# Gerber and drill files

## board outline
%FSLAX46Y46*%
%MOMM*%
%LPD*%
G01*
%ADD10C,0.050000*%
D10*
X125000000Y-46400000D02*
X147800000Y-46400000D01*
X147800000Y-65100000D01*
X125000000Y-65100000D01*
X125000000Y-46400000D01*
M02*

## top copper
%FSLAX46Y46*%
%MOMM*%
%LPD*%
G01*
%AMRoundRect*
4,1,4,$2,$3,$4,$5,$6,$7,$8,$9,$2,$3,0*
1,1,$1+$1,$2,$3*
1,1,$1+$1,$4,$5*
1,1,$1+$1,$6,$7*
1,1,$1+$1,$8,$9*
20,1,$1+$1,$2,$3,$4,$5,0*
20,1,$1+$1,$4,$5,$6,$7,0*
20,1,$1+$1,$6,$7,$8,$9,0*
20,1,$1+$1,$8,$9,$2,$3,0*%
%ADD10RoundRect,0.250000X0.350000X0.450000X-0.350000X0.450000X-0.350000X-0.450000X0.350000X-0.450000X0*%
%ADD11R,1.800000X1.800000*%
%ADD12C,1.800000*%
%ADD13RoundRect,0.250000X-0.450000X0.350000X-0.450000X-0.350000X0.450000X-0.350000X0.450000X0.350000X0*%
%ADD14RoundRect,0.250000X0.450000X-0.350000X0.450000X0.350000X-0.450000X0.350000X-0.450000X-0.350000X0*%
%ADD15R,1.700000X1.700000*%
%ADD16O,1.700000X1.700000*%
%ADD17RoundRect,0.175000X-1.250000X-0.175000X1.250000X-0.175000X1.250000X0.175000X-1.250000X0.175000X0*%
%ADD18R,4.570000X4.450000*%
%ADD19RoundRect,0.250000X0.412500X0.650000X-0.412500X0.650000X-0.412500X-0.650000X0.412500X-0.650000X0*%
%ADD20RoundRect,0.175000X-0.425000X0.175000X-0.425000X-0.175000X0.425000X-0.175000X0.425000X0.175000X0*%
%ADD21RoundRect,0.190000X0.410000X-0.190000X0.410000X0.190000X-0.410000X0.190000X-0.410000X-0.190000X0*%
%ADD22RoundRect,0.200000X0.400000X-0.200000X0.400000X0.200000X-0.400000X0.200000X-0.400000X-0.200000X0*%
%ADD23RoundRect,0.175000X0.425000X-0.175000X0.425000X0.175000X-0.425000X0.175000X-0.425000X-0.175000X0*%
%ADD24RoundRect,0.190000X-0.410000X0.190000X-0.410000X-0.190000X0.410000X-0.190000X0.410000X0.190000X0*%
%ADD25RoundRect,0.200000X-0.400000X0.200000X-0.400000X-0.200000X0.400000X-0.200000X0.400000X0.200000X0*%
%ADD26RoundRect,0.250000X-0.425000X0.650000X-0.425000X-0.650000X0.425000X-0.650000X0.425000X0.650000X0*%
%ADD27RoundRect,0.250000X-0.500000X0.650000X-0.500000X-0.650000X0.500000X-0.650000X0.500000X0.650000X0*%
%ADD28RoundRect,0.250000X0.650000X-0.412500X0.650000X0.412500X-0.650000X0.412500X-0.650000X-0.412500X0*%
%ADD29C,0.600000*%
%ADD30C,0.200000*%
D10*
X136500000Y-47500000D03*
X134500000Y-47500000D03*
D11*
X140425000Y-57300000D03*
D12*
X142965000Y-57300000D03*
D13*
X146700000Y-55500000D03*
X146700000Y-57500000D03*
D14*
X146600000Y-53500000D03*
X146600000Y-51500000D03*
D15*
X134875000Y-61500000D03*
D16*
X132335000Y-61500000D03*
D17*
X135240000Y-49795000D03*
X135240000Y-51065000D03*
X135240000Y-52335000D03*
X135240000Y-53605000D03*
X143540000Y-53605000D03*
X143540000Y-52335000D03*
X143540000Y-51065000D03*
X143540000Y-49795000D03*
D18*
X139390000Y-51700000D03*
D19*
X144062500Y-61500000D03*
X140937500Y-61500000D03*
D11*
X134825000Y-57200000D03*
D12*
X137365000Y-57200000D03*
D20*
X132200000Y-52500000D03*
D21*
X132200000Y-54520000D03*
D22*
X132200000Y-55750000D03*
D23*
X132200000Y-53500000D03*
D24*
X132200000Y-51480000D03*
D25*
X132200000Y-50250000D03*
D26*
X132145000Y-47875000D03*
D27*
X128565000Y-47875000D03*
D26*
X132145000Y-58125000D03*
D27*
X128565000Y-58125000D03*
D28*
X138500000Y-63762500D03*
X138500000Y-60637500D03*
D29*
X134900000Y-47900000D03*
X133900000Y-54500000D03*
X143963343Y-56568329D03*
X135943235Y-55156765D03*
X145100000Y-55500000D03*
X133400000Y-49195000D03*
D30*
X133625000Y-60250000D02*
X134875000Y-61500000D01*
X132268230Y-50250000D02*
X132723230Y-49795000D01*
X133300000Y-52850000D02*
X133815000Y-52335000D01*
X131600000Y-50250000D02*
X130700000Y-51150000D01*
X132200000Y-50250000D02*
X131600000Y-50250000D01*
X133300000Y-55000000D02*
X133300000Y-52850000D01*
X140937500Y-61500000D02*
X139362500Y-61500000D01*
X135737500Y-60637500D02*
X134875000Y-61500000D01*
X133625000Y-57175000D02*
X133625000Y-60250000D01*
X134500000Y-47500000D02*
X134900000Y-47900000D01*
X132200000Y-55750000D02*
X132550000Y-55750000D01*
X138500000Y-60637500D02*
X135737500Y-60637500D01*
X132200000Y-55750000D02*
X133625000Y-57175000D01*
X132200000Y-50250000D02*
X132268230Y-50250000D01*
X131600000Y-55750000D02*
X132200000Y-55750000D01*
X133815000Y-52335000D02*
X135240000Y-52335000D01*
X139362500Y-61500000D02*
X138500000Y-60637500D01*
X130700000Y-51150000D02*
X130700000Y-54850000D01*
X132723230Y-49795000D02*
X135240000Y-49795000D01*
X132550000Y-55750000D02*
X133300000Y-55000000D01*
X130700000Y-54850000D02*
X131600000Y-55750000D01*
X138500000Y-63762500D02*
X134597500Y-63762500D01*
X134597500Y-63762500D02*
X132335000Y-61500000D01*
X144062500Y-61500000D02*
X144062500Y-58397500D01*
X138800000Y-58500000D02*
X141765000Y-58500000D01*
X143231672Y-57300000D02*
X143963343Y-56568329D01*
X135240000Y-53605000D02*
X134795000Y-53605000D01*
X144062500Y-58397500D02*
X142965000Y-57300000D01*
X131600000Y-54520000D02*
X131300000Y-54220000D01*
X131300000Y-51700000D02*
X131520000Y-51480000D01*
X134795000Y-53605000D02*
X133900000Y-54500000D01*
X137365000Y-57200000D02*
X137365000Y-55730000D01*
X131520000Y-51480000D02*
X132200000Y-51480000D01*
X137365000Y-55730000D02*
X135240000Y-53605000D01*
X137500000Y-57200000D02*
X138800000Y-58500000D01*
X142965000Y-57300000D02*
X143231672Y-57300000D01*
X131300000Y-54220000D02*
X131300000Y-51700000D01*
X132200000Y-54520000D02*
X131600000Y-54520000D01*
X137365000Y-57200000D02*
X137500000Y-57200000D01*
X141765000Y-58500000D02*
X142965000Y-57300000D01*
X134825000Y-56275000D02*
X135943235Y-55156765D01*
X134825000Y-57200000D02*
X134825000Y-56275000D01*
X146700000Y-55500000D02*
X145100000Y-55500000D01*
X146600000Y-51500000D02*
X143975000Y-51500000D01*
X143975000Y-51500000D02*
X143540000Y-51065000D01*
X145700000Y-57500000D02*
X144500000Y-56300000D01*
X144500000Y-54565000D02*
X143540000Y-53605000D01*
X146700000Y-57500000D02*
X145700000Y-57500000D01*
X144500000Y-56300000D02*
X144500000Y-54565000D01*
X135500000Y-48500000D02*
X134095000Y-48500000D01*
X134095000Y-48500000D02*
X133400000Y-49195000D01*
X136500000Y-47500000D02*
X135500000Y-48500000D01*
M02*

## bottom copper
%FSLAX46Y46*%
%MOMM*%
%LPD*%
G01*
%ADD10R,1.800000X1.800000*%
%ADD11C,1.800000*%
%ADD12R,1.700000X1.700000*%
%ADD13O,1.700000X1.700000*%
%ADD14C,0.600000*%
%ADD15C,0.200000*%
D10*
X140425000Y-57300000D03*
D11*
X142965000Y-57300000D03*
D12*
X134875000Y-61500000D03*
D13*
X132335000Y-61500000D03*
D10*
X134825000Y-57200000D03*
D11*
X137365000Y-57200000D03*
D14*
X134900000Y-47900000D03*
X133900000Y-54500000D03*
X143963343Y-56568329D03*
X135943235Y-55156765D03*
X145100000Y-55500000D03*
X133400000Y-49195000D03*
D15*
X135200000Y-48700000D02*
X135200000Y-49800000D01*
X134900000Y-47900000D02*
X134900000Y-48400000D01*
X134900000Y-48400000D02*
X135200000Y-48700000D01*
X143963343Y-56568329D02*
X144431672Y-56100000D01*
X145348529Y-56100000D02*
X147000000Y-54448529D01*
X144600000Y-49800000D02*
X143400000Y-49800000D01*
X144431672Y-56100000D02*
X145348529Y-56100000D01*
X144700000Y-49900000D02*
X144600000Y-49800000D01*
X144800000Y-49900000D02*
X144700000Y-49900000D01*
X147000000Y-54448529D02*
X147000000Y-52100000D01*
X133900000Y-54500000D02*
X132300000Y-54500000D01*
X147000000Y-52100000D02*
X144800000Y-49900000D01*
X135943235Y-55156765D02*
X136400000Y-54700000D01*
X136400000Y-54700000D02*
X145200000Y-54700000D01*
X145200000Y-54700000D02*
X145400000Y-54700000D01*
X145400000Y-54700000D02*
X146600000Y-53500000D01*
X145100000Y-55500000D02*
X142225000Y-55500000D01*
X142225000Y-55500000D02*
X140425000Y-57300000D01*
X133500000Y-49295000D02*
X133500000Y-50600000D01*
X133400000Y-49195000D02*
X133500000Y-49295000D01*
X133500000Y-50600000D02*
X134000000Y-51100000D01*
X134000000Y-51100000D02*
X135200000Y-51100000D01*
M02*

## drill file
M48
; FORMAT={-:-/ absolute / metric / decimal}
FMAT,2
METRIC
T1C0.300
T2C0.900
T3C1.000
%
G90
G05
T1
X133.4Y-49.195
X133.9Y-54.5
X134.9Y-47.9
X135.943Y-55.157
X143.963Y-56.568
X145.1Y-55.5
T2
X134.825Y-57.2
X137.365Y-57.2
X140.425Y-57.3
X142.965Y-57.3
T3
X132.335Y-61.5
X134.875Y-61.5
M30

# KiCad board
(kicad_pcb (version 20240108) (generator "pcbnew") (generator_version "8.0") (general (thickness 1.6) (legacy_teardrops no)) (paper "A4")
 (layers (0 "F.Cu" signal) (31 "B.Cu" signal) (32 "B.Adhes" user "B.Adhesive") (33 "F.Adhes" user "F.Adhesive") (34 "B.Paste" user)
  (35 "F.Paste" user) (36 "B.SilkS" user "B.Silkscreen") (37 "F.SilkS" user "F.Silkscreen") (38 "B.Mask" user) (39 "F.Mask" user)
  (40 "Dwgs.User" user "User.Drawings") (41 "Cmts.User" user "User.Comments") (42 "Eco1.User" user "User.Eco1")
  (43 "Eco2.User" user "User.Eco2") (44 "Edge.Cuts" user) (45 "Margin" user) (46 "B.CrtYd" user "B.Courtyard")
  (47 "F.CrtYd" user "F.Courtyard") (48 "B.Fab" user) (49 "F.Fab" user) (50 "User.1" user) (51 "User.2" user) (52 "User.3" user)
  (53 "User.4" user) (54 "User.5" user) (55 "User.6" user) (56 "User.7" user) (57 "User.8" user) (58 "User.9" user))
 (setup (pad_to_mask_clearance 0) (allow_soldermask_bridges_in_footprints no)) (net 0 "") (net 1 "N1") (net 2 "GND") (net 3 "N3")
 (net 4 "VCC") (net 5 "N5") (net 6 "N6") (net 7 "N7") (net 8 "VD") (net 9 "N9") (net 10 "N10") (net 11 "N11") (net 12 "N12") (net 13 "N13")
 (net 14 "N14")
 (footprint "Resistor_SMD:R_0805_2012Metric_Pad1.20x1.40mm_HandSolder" (layer "F.Cu") (at 135.5 47.5 180)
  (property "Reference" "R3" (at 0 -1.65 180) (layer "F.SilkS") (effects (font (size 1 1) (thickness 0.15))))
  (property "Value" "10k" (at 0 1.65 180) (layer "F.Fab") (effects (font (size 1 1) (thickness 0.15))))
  (pad "1" smd roundrect (at -1 0 180) (size 1.2 1.4) (layers "F.Cu" "F.Paste" "F.Mask") (roundrect_rratio 0.208333) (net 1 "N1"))
  (pad "2" smd roundrect (at 1 0 180) (size 1.2 1.4) (layers "F.Cu" "F.Paste" "F.Mask") (roundrect_rratio 0.208333) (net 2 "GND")))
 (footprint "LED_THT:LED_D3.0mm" (layer "F.Cu") (at 140.425 57.3)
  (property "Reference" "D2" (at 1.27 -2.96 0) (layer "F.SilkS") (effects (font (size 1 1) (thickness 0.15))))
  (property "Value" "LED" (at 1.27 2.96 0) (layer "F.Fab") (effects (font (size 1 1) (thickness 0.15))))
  (pad "1" thru_hole rect (at 0 0) (size 1.8 1.8) (drill 0.9) (layers "*.Cu" "*.Mask") (remove_unused_layers no) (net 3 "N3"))
  (pad "2" thru_hole circle (at 2.54 0) (size 1.8 1.8) (drill 0.9) (layers "*.Cu" "*.Mask") (remove_unused_layers no) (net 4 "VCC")))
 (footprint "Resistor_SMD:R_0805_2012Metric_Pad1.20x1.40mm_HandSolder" (layer "F.Cu") (at 146.7 56.5 -90)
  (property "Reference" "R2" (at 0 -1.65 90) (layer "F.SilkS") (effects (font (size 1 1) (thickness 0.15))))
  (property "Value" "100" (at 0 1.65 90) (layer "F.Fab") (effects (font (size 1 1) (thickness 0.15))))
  (pad "1" smd roundrect (at -1 0 270) (size 1.2 1.4) (layers "F.Cu" "F.Paste" "F.Mask") (roundrect_rratio 0.208333) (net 3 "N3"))
  (pad "2" smd roundrect (at 1 0 270) (size 1.2 1.4) (layers "F.Cu" "F.Paste" "F.Mask") (roundrect_rratio 0.208333) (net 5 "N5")))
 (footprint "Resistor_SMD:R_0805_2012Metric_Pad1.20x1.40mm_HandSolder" (layer "F.Cu") (at 146.6 52.5 90)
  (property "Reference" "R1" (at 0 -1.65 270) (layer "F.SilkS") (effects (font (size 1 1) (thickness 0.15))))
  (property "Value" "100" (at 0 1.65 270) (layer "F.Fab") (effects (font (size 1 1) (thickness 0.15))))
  (pad "1" smd roundrect (at -1 0 90) (size 1.2 1.4) (layers "F.Cu" "F.Paste" "F.Mask") (roundrect_rratio 0.208333) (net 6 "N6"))
  (pad "2" smd roundrect (at 1 0 90) (size 1.2 1.4) (layers "F.Cu" "F.Paste" "F.Mask") (roundrect_rratio 0.208333) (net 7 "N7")))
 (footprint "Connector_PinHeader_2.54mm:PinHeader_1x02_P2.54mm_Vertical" (layer "F.Cu") (at 134.875 61.5 -90)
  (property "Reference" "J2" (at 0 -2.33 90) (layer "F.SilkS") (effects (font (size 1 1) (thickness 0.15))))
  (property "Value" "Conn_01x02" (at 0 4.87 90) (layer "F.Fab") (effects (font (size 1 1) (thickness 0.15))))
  (pad "1" thru_hole rect (at 0 0 270) (size 1.7 1.7) (drill 1) (layers "*.Cu" "*.Mask") (remove_unused_layers no) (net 2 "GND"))
  (pad "2" thru_hole oval (at 0 2.54 270) (size 1.7 1.7) (drill 1) (layers "*.Cu" "*.Mask") (remove_unused_layers no) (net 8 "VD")))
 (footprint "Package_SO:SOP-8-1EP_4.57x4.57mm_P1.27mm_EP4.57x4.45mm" (layer "F.Cu") (at 139.39 51.7)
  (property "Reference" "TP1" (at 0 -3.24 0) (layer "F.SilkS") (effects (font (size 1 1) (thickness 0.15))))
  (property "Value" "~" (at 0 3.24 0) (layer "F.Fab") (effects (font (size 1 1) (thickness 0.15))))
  (pad "" smd roundrect (at -1.14 -1.11) (size 1.84 1.79) (layers "F.Paste") (roundrect_rratio 0.139665))
  (pad "" smd roundrect (at -1.14 1.11) (size 1.84 1.79) (layers "F.Paste") (roundrect_rratio 0.139665))
  (pad "" smd roundrect (at 1.14 -1.11) (size 1.84 1.79) (layers "F.Paste") (roundrect_rratio 0.139665))
  (pad "" smd roundrect (at 1.14 1.11) (size 1.84 1.79) (layers "F.Paste") (roundrect_rratio 0.139665))
  (pad "1" smd roundrect (at -4.15 -1.905) (size 2.85 0.7) (layers "F.Cu" "F.Paste" "F.Mask") (roundrect_rratio 0.25) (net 2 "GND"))
  (pad "2" smd roundrect (at -4.15 -0.635) (size 2.85 0.7) (layers "F.Cu" "F.Paste" "F.Mask") (roundrect_rratio 0.25) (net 1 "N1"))
  (pad "3" smd roundrect (at -4.15 0.635) (size 2.85 0.7) (layers "F.Cu" "F.Paste" "F.Mask") (roundrect_rratio 0.25) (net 2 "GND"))
  (pad "4" smd roundrect (at -4.15 1.905) (size 2.85 0.7) (layers "F.Cu" "F.Paste" "F.Mask") (roundrect_rratio 0.25) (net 4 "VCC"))
  (pad "5" smd roundrect (at 4.15 1.905) (size 2.85 0.7) (layers "F.Cu" "F.Paste" "F.Mask") (roundrect_rratio 0.25) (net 5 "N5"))
  (pad "6" smd roundrect (at 4.15 0.635) (size 2.85 0.7) (layers "F.Cu" "F.Paste" "F.Mask") (roundrect_rratio 0.25))
  (pad "7" smd roundrect (at 4.15 -0.635) (size 2.85 0.7) (layers "F.Cu" "F.Paste" "F.Mask") (roundrect_rratio 0.25) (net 7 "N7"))
  (pad "8" smd roundrect (at 4.15 -1.905) (size 2.85 0.7) (layers "F.Cu" "F.Paste" "F.Mask") (roundrect_rratio 0.25) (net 4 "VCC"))
  (pad "9" smd rect (at 0 0) (size 4.57 4.45) (layers "F.Cu" "F.Mask") (zone_connect 2)))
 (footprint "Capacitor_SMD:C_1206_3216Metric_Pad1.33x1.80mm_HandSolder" (layer "F.Cu") (at 142.5 61.5 180)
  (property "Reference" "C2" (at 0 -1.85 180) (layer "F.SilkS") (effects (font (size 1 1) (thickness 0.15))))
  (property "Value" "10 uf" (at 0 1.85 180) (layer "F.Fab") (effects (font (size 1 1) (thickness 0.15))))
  (pad "1" smd roundrect (at -1.5625 0 180) (size 1.325 1.8) (layers "F.Cu" "F.Paste" "F.Mask") (roundrect_rratio 0.188679) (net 4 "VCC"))
  (pad "2" smd roundrect (at 1.5625 0 180) (size 1.325 1.8) (layers "F.Cu" "F.Paste" "F.Mask") (roundrect_rratio 0.188679) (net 2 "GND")))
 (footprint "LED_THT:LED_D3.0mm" (layer "F.Cu") (at 134.825 57.2)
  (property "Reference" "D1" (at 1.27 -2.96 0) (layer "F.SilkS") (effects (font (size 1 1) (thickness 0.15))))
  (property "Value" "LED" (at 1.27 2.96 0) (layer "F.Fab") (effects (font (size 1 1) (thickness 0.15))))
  (pad "1" thru_hole rect (at 0 0) (size 1.8 1.8) (drill 0.9) (layers "*.Cu" "*.Mask") (remove_unused_layers no) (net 6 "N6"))
  (pad "2" thru_hole circle (at 2.54 0) (size 1.8 1.8) (drill 0.9) (layers "*.Cu" "*.Mask") (remove_unused_layers no) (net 4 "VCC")))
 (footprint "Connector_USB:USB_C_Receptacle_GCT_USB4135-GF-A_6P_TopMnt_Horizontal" (layer "F.Cu") (at 129.1675 53 -90)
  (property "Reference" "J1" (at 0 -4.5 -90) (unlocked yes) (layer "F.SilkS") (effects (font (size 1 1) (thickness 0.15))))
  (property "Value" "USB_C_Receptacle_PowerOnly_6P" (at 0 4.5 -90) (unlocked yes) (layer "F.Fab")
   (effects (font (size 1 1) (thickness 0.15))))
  (pad "A5" smd roundrect (at -0.5 -3.0325 270) (size 0.7 1.2) (layers "F.Cu" "F.Paste" "F.Mask") (roundrect_rratio 0.25) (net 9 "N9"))
  (pad "A9" smd roundrect (at 1.52 -3.0325 90) (size 0.76 1.2) (layers "F.Cu" "F.Paste" "F.Mask") (roundrect_rratio 0.25) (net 4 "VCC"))
  (pad "A12" smd roundrect (at 2.75 -3.0325 90) (size 0.8 1.2) (layers "F.Cu" "F.Paste" "F.Mask") (roundrect_rratio 0.25) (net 2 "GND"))
  (pad "B5" smd roundrect (at 0.5 -3.0325 90) (size 0.7 1.2) (layers "F.Cu" "F.Paste" "F.Mask") (roundrect_rratio 0.25) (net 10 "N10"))
  (pad "B9" smd roundrect (at -1.52 -3.0325 270) (size 0.76 1.2) (layers "F.Cu" "F.Paste" "F.Mask") (roundrect_rratio 0.25) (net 4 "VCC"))
  (pad "B12" smd roundrect (at -2.75 -3.0325 270) (size 0.8 1.2) (layers "F.Cu" "F.Paste" "F.Mask") (roundrect_rratio 0.25) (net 2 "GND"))
  (pad "S1" smd roundrect (at -5.125 -2.9775 270) (size 1.8 1.35) (layers "F.Cu" "F.Paste" "F.Mask") (roundrect_rratio 0.1851851852)
   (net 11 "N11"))
  (pad "S1" smd roundrect (at -5.125 0.6025 270) (size 1.8 1.5) (layers "F.Cu" "F.Paste" "F.Mask") (roundrect_rratio 0.1666666667)
   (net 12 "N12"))
  (pad "S1" smd roundrect (at 5.125 -2.9775 270) (size 1.8 1.35) (layers "F.Cu" "F.Paste" "F.Mask") (roundrect_rratio 0.1851851852)
   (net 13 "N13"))
  (pad "S1" smd roundrect (at 5.125 0.6025 270) (size 1.8 1.5) (layers "F.Cu" "F.Paste" "F.Mask") (roundrect_rratio 0.1666666667)
   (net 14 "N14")))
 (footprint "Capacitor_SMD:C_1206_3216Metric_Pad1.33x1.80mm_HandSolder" (layer "F.Cu") (at 138.5 62.2 90)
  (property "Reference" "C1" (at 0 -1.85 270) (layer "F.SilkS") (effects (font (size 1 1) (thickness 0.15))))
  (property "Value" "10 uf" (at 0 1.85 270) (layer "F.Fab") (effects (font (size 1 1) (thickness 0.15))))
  (pad "1" smd roundrect (at -1.5625 0 90) (size 1.325 1.8) (layers "F.Cu" "F.Paste" "F.Mask") (roundrect_rratio 0.188679) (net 8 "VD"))
  (pad "2" smd roundrect (at 1.5625 0 90) (size 1.325 1.8) (layers "F.Cu" "F.Paste" "F.Mask") (roundrect_rratio 0.188679) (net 2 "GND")))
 (gr_rect (start 125 46.4) (end 147.8 65.1) (stroke (width 0.05) (type default)) (fill none) (layer "Edge.Cuts"))
 (segment (start 133.625 60.25) (end 134.875 61.5) (width 0.2) (layer "F.Cu") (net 2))
 (segment (start 132.26823 50.25) (end 132.72323 49.795) (width 0.2) (layer "F.Cu") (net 2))
 (segment (start 133.3 52.85) (end 133.815 52.335) (width 0.2) (layer "F.Cu") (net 2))
 (segment (start 131.6 50.25) (end 130.7 51.15) (width 0.2) (layer "F.Cu") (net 2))
 (segment (start 132.2 50.25) (end 131.6 50.25) (width 0.2) (layer "F.Cu") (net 2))
 (segment (start 133.3 55) (end 133.3 52.85) (width 0.2) (layer "F.Cu") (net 2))
 (segment (start 140.9375 61.5) (end 139.3625 61.5) (width 0.2) (layer "F.Cu") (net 2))
 (segment (start 135.7375 60.6375) (end 134.875 61.5) (width 0.2) (layer "F.Cu") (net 2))
 (segment (start 133.625 57.175) (end 133.625 60.25) (width 0.2) (layer "F.Cu") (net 2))
 (segment (start 134.5 47.5) (end 134.9 47.9) (width 0.2) (layer "F.Cu") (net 2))
 (segment (start 132.2 55.75) (end 132.55 55.75) (width 0.2) (layer "F.Cu") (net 2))
 (segment (start 138.5 60.6375) (end 135.7375 60.6375) (width 0.2) (layer "F.Cu") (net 2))
 (segment (start 132.2 55.75) (end 133.625 57.175) (width 0.2) (layer "F.Cu") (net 2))
 (segment (start 132.2 50.25) (end 132.26823 50.25) (width 0.2) (layer "F.Cu") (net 2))
 (segment (start 131.6 55.75) (end 132.2 55.75) (width 0.2) (layer "F.Cu") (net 2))
 (segment (start 133.815 52.335) (end 135.24 52.335) (width 0.2) (layer "F.Cu") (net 2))
 (segment (start 139.3625 61.5) (end 138.5 60.6375) (width 0.2) (layer "F.Cu") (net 2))
 (segment (start 130.7 51.15) (end 130.7 54.85) (width 0.2) (layer "F.Cu") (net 2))
 (segment (start 132.72323 49.795) (end 135.24 49.795) (width 0.2) (layer "F.Cu") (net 2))
 (segment (start 132.55 55.75) (end 133.3 55) (width 0.2) (layer "F.Cu") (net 2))
 (segment (start 130.7 54.85) (end 131.6 55.75) (width 0.2) (layer "F.Cu") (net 2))
 (via (at 134.9 47.9) (size 0.6) (drill 0.3) (layers "F.Cu" "B.Cu") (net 2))
 (segment (start 135.2 48.7) (end 135.2 49.8) (width 0.2) (layer "B.Cu") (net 2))
 (segment (start 134.9 47.9) (end 134.9 48.4) (width 0.2) (layer "B.Cu") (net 2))
 (segment (start 134.9 48.4) (end 135.2 48.7) (width 0.2) (layer "B.Cu") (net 2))
 (segment (start 138.5 63.7625) (end 134.5975 63.7625) (width 0.2) (layer "F.Cu") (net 8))
 (segment (start 134.5975 63.7625) (end 132.335 61.5) (width 0.2) (layer "F.Cu") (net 8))
 (segment (start 144.0625 61.5) (end 144.0625 58.3975) (width 0.2) (layer "F.Cu") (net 4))
 (segment (start 138.8 58.5) (end 141.765 58.5) (width 0.2) (layer "F.Cu") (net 4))
 (segment (start 143.231672 57.3) (end 143.963343 56.568329) (width 0.2) (layer "F.Cu") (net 4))
 (segment (start 135.24 53.605) (end 134.795 53.605) (width 0.2) (layer "F.Cu") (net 4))
 (segment (start 144.0625 58.3975) (end 142.965 57.3) (width 0.2) (layer "F.Cu") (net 4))
 (segment (start 131.6 54.52) (end 131.3 54.22) (width 0.2) (layer "F.Cu") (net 4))
 (segment (start 131.3 51.7) (end 131.52 51.48) (width 0.2) (layer "F.Cu") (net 4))
 (segment (start 134.795 53.605) (end 133.9 54.5) (width 0.2) (layer "F.Cu") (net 4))
 (segment (start 137.365 57.2) (end 137.365 55.73) (width 0.2) (layer "F.Cu") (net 4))
 (segment (start 131.52 51.48) (end 132.2 51.48) (width 0.2) (layer "F.Cu") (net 4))
 (segment (start 137.365 55.73) (end 135.24 53.605) (width 0.2) (layer "F.Cu") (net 4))
 (segment (start 137.5 57.2) (end 138.8 58.5) (width 0.2) (layer "F.Cu") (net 4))
 (segment (start 142.965 57.3) (end 143.231672 57.3) (width 0.2) (layer "F.Cu") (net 4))
 (segment (start 131.3 54.22) (end 131.3 51.7) (width 0.2) (layer "F.Cu") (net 4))
 (segment (start 132.2 54.52) (end 131.6 54.52) (width 0.2) (layer "F.Cu") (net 4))
 (segment (start 137.365 57.2) (end 137.5 57.2) (width 0.2) (layer "F.Cu") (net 4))
 (segment (start 141.765 58.5) (end 142.965 57.3) (width 0.2) (layer "F.Cu") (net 4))
 (via (at 133.9 54.5) (size 0.6) (drill 0.3) (layers "F.Cu" "B.Cu") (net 4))
 (via (at 143.963343 56.568329) (size 0.6) (drill 0.3) (layers "F.Cu" "B.Cu") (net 4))
 (segment (start 143.963343 56.568329) (end 144.431672 56.1) (width 0.2) (layer "B.Cu") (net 4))
 (segment (start 145.348529 56.1) (end 147 54.448529) (width 0.2) (layer "B.Cu") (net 4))
 (segment (start 144.6 49.8) (end 143.4 49.8) (width 0.2) (layer "B.Cu") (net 4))
 (segment (start 144.431672 56.1) (end 145.348529 56.1) (width 0.2) (layer "B.Cu") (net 4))
 (segment (start 144.7 49.9) (end 144.6 49.8) (width 0.2) (layer "B.Cu") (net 4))
 (segment (start 144.8 49.9) (end 144.7 49.9) (width 0.2) (layer "B.Cu") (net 4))
 (segment (start 147 54.448529) (end 147 52.1) (width 0.2) (layer "B.Cu") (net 4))
 (segment (start 133.9 54.5) (end 132.3 54.5) (width 0.2) (layer "B.Cu") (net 4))
 (segment (start 147 52.1) (end 144.8 49.9) (width 0.2) (layer "B.Cu") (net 4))
 (segment (start 134.825 56.275) (end 135.943235 55.156765) (width 0.2) (layer "F.Cu") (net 6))
 (segment (start 134.825 57.2) (end 134.825 56.275) (width 0.2) (layer "F.Cu") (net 6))
 (via (at 135.943235 55.156765) (size 0.6) (drill 0.3) (layers "F.Cu" "B.Cu") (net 6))
 (segment (start 135.943235 55.156765) (end 136.4 54.7) (width 0.2) (layer "B.Cu") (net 6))
 (segment (start 136.4 54.7) (end 145.2 54.7) (width 0.2) (layer "B.Cu") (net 6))
 (segment (start 145.2 54.7) (end 145.4 54.7) (width 0.2) (layer "B.Cu") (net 6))
 (segment (start 145.4 54.7) (end 146.6 53.5) (width 0.2) (layer "B.Cu") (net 6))
 (segment (start 146.7 55.5) (end 145.1 55.5) (width 0.2) (layer "F.Cu") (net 3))
 (via (at 145.1 55.5) (size 0.6) (drill 0.3) (layers "F.Cu" "B.Cu") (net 3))
 (segment (start 145.1 55.5) (end 142.225 55.5) (width 0.2) (layer "B.Cu") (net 3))
 (segment (start 142.225 55.5) (end 140.425 57.3) (width 0.2) (layer "B.Cu") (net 3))
 (segment (start 146.6 51.5) (end 143.975 51.5) (width 0.2) (layer "F.Cu") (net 7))
 (segment (start 143.975 51.5) (end 143.54 51.065) (width 0.2) (layer "F.Cu") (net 7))
 (segment (start 145.7 57.5) (end 144.5 56.3) (width 0.2) (layer "F.Cu") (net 5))
 (segment (start 144.5 54.565) (end 143.54 53.605) (width 0.2) (layer "F.Cu") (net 5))
 (segment (start 146.7 57.5) (end 145.7 57.5) (width 0.2) (layer "F.Cu") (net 5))
 (segment (start 144.5 56.3) (end 144.5 54.565) (width 0.2) (layer "F.Cu") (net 5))
 (segment (start 135.5 48.5) (end 134.095 48.5) (width 0.2) (layer "F.Cu") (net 1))
 (segment (start 134.095 48.5) (end 133.4 49.195) (width 0.2) (layer "F.Cu") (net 1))
 (segment (start 136.5 47.5) (end 135.5 48.5) (width 0.2) (layer "F.Cu") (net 1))
 (via (at 133.4 49.195) (size 0.6) (drill 0.3) (layers "F.Cu" "B.Cu") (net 1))
 (segment (start 133.5 49.295) (end 133.5 50.6) (width 0.2) (layer "B.Cu") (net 1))
 (segment (start 133.4 49.195) (end 133.5 49.295) (width 0.2) (layer "B.Cu") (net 1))
 (segment (start 133.5 50.6) (end 134 51.1) (width 0.2) (layer "B.Cu") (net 1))
 (segment (start 134 51.1) (end 135.2 51.1) (width 0.2) (layer "B.Cu") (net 1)))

